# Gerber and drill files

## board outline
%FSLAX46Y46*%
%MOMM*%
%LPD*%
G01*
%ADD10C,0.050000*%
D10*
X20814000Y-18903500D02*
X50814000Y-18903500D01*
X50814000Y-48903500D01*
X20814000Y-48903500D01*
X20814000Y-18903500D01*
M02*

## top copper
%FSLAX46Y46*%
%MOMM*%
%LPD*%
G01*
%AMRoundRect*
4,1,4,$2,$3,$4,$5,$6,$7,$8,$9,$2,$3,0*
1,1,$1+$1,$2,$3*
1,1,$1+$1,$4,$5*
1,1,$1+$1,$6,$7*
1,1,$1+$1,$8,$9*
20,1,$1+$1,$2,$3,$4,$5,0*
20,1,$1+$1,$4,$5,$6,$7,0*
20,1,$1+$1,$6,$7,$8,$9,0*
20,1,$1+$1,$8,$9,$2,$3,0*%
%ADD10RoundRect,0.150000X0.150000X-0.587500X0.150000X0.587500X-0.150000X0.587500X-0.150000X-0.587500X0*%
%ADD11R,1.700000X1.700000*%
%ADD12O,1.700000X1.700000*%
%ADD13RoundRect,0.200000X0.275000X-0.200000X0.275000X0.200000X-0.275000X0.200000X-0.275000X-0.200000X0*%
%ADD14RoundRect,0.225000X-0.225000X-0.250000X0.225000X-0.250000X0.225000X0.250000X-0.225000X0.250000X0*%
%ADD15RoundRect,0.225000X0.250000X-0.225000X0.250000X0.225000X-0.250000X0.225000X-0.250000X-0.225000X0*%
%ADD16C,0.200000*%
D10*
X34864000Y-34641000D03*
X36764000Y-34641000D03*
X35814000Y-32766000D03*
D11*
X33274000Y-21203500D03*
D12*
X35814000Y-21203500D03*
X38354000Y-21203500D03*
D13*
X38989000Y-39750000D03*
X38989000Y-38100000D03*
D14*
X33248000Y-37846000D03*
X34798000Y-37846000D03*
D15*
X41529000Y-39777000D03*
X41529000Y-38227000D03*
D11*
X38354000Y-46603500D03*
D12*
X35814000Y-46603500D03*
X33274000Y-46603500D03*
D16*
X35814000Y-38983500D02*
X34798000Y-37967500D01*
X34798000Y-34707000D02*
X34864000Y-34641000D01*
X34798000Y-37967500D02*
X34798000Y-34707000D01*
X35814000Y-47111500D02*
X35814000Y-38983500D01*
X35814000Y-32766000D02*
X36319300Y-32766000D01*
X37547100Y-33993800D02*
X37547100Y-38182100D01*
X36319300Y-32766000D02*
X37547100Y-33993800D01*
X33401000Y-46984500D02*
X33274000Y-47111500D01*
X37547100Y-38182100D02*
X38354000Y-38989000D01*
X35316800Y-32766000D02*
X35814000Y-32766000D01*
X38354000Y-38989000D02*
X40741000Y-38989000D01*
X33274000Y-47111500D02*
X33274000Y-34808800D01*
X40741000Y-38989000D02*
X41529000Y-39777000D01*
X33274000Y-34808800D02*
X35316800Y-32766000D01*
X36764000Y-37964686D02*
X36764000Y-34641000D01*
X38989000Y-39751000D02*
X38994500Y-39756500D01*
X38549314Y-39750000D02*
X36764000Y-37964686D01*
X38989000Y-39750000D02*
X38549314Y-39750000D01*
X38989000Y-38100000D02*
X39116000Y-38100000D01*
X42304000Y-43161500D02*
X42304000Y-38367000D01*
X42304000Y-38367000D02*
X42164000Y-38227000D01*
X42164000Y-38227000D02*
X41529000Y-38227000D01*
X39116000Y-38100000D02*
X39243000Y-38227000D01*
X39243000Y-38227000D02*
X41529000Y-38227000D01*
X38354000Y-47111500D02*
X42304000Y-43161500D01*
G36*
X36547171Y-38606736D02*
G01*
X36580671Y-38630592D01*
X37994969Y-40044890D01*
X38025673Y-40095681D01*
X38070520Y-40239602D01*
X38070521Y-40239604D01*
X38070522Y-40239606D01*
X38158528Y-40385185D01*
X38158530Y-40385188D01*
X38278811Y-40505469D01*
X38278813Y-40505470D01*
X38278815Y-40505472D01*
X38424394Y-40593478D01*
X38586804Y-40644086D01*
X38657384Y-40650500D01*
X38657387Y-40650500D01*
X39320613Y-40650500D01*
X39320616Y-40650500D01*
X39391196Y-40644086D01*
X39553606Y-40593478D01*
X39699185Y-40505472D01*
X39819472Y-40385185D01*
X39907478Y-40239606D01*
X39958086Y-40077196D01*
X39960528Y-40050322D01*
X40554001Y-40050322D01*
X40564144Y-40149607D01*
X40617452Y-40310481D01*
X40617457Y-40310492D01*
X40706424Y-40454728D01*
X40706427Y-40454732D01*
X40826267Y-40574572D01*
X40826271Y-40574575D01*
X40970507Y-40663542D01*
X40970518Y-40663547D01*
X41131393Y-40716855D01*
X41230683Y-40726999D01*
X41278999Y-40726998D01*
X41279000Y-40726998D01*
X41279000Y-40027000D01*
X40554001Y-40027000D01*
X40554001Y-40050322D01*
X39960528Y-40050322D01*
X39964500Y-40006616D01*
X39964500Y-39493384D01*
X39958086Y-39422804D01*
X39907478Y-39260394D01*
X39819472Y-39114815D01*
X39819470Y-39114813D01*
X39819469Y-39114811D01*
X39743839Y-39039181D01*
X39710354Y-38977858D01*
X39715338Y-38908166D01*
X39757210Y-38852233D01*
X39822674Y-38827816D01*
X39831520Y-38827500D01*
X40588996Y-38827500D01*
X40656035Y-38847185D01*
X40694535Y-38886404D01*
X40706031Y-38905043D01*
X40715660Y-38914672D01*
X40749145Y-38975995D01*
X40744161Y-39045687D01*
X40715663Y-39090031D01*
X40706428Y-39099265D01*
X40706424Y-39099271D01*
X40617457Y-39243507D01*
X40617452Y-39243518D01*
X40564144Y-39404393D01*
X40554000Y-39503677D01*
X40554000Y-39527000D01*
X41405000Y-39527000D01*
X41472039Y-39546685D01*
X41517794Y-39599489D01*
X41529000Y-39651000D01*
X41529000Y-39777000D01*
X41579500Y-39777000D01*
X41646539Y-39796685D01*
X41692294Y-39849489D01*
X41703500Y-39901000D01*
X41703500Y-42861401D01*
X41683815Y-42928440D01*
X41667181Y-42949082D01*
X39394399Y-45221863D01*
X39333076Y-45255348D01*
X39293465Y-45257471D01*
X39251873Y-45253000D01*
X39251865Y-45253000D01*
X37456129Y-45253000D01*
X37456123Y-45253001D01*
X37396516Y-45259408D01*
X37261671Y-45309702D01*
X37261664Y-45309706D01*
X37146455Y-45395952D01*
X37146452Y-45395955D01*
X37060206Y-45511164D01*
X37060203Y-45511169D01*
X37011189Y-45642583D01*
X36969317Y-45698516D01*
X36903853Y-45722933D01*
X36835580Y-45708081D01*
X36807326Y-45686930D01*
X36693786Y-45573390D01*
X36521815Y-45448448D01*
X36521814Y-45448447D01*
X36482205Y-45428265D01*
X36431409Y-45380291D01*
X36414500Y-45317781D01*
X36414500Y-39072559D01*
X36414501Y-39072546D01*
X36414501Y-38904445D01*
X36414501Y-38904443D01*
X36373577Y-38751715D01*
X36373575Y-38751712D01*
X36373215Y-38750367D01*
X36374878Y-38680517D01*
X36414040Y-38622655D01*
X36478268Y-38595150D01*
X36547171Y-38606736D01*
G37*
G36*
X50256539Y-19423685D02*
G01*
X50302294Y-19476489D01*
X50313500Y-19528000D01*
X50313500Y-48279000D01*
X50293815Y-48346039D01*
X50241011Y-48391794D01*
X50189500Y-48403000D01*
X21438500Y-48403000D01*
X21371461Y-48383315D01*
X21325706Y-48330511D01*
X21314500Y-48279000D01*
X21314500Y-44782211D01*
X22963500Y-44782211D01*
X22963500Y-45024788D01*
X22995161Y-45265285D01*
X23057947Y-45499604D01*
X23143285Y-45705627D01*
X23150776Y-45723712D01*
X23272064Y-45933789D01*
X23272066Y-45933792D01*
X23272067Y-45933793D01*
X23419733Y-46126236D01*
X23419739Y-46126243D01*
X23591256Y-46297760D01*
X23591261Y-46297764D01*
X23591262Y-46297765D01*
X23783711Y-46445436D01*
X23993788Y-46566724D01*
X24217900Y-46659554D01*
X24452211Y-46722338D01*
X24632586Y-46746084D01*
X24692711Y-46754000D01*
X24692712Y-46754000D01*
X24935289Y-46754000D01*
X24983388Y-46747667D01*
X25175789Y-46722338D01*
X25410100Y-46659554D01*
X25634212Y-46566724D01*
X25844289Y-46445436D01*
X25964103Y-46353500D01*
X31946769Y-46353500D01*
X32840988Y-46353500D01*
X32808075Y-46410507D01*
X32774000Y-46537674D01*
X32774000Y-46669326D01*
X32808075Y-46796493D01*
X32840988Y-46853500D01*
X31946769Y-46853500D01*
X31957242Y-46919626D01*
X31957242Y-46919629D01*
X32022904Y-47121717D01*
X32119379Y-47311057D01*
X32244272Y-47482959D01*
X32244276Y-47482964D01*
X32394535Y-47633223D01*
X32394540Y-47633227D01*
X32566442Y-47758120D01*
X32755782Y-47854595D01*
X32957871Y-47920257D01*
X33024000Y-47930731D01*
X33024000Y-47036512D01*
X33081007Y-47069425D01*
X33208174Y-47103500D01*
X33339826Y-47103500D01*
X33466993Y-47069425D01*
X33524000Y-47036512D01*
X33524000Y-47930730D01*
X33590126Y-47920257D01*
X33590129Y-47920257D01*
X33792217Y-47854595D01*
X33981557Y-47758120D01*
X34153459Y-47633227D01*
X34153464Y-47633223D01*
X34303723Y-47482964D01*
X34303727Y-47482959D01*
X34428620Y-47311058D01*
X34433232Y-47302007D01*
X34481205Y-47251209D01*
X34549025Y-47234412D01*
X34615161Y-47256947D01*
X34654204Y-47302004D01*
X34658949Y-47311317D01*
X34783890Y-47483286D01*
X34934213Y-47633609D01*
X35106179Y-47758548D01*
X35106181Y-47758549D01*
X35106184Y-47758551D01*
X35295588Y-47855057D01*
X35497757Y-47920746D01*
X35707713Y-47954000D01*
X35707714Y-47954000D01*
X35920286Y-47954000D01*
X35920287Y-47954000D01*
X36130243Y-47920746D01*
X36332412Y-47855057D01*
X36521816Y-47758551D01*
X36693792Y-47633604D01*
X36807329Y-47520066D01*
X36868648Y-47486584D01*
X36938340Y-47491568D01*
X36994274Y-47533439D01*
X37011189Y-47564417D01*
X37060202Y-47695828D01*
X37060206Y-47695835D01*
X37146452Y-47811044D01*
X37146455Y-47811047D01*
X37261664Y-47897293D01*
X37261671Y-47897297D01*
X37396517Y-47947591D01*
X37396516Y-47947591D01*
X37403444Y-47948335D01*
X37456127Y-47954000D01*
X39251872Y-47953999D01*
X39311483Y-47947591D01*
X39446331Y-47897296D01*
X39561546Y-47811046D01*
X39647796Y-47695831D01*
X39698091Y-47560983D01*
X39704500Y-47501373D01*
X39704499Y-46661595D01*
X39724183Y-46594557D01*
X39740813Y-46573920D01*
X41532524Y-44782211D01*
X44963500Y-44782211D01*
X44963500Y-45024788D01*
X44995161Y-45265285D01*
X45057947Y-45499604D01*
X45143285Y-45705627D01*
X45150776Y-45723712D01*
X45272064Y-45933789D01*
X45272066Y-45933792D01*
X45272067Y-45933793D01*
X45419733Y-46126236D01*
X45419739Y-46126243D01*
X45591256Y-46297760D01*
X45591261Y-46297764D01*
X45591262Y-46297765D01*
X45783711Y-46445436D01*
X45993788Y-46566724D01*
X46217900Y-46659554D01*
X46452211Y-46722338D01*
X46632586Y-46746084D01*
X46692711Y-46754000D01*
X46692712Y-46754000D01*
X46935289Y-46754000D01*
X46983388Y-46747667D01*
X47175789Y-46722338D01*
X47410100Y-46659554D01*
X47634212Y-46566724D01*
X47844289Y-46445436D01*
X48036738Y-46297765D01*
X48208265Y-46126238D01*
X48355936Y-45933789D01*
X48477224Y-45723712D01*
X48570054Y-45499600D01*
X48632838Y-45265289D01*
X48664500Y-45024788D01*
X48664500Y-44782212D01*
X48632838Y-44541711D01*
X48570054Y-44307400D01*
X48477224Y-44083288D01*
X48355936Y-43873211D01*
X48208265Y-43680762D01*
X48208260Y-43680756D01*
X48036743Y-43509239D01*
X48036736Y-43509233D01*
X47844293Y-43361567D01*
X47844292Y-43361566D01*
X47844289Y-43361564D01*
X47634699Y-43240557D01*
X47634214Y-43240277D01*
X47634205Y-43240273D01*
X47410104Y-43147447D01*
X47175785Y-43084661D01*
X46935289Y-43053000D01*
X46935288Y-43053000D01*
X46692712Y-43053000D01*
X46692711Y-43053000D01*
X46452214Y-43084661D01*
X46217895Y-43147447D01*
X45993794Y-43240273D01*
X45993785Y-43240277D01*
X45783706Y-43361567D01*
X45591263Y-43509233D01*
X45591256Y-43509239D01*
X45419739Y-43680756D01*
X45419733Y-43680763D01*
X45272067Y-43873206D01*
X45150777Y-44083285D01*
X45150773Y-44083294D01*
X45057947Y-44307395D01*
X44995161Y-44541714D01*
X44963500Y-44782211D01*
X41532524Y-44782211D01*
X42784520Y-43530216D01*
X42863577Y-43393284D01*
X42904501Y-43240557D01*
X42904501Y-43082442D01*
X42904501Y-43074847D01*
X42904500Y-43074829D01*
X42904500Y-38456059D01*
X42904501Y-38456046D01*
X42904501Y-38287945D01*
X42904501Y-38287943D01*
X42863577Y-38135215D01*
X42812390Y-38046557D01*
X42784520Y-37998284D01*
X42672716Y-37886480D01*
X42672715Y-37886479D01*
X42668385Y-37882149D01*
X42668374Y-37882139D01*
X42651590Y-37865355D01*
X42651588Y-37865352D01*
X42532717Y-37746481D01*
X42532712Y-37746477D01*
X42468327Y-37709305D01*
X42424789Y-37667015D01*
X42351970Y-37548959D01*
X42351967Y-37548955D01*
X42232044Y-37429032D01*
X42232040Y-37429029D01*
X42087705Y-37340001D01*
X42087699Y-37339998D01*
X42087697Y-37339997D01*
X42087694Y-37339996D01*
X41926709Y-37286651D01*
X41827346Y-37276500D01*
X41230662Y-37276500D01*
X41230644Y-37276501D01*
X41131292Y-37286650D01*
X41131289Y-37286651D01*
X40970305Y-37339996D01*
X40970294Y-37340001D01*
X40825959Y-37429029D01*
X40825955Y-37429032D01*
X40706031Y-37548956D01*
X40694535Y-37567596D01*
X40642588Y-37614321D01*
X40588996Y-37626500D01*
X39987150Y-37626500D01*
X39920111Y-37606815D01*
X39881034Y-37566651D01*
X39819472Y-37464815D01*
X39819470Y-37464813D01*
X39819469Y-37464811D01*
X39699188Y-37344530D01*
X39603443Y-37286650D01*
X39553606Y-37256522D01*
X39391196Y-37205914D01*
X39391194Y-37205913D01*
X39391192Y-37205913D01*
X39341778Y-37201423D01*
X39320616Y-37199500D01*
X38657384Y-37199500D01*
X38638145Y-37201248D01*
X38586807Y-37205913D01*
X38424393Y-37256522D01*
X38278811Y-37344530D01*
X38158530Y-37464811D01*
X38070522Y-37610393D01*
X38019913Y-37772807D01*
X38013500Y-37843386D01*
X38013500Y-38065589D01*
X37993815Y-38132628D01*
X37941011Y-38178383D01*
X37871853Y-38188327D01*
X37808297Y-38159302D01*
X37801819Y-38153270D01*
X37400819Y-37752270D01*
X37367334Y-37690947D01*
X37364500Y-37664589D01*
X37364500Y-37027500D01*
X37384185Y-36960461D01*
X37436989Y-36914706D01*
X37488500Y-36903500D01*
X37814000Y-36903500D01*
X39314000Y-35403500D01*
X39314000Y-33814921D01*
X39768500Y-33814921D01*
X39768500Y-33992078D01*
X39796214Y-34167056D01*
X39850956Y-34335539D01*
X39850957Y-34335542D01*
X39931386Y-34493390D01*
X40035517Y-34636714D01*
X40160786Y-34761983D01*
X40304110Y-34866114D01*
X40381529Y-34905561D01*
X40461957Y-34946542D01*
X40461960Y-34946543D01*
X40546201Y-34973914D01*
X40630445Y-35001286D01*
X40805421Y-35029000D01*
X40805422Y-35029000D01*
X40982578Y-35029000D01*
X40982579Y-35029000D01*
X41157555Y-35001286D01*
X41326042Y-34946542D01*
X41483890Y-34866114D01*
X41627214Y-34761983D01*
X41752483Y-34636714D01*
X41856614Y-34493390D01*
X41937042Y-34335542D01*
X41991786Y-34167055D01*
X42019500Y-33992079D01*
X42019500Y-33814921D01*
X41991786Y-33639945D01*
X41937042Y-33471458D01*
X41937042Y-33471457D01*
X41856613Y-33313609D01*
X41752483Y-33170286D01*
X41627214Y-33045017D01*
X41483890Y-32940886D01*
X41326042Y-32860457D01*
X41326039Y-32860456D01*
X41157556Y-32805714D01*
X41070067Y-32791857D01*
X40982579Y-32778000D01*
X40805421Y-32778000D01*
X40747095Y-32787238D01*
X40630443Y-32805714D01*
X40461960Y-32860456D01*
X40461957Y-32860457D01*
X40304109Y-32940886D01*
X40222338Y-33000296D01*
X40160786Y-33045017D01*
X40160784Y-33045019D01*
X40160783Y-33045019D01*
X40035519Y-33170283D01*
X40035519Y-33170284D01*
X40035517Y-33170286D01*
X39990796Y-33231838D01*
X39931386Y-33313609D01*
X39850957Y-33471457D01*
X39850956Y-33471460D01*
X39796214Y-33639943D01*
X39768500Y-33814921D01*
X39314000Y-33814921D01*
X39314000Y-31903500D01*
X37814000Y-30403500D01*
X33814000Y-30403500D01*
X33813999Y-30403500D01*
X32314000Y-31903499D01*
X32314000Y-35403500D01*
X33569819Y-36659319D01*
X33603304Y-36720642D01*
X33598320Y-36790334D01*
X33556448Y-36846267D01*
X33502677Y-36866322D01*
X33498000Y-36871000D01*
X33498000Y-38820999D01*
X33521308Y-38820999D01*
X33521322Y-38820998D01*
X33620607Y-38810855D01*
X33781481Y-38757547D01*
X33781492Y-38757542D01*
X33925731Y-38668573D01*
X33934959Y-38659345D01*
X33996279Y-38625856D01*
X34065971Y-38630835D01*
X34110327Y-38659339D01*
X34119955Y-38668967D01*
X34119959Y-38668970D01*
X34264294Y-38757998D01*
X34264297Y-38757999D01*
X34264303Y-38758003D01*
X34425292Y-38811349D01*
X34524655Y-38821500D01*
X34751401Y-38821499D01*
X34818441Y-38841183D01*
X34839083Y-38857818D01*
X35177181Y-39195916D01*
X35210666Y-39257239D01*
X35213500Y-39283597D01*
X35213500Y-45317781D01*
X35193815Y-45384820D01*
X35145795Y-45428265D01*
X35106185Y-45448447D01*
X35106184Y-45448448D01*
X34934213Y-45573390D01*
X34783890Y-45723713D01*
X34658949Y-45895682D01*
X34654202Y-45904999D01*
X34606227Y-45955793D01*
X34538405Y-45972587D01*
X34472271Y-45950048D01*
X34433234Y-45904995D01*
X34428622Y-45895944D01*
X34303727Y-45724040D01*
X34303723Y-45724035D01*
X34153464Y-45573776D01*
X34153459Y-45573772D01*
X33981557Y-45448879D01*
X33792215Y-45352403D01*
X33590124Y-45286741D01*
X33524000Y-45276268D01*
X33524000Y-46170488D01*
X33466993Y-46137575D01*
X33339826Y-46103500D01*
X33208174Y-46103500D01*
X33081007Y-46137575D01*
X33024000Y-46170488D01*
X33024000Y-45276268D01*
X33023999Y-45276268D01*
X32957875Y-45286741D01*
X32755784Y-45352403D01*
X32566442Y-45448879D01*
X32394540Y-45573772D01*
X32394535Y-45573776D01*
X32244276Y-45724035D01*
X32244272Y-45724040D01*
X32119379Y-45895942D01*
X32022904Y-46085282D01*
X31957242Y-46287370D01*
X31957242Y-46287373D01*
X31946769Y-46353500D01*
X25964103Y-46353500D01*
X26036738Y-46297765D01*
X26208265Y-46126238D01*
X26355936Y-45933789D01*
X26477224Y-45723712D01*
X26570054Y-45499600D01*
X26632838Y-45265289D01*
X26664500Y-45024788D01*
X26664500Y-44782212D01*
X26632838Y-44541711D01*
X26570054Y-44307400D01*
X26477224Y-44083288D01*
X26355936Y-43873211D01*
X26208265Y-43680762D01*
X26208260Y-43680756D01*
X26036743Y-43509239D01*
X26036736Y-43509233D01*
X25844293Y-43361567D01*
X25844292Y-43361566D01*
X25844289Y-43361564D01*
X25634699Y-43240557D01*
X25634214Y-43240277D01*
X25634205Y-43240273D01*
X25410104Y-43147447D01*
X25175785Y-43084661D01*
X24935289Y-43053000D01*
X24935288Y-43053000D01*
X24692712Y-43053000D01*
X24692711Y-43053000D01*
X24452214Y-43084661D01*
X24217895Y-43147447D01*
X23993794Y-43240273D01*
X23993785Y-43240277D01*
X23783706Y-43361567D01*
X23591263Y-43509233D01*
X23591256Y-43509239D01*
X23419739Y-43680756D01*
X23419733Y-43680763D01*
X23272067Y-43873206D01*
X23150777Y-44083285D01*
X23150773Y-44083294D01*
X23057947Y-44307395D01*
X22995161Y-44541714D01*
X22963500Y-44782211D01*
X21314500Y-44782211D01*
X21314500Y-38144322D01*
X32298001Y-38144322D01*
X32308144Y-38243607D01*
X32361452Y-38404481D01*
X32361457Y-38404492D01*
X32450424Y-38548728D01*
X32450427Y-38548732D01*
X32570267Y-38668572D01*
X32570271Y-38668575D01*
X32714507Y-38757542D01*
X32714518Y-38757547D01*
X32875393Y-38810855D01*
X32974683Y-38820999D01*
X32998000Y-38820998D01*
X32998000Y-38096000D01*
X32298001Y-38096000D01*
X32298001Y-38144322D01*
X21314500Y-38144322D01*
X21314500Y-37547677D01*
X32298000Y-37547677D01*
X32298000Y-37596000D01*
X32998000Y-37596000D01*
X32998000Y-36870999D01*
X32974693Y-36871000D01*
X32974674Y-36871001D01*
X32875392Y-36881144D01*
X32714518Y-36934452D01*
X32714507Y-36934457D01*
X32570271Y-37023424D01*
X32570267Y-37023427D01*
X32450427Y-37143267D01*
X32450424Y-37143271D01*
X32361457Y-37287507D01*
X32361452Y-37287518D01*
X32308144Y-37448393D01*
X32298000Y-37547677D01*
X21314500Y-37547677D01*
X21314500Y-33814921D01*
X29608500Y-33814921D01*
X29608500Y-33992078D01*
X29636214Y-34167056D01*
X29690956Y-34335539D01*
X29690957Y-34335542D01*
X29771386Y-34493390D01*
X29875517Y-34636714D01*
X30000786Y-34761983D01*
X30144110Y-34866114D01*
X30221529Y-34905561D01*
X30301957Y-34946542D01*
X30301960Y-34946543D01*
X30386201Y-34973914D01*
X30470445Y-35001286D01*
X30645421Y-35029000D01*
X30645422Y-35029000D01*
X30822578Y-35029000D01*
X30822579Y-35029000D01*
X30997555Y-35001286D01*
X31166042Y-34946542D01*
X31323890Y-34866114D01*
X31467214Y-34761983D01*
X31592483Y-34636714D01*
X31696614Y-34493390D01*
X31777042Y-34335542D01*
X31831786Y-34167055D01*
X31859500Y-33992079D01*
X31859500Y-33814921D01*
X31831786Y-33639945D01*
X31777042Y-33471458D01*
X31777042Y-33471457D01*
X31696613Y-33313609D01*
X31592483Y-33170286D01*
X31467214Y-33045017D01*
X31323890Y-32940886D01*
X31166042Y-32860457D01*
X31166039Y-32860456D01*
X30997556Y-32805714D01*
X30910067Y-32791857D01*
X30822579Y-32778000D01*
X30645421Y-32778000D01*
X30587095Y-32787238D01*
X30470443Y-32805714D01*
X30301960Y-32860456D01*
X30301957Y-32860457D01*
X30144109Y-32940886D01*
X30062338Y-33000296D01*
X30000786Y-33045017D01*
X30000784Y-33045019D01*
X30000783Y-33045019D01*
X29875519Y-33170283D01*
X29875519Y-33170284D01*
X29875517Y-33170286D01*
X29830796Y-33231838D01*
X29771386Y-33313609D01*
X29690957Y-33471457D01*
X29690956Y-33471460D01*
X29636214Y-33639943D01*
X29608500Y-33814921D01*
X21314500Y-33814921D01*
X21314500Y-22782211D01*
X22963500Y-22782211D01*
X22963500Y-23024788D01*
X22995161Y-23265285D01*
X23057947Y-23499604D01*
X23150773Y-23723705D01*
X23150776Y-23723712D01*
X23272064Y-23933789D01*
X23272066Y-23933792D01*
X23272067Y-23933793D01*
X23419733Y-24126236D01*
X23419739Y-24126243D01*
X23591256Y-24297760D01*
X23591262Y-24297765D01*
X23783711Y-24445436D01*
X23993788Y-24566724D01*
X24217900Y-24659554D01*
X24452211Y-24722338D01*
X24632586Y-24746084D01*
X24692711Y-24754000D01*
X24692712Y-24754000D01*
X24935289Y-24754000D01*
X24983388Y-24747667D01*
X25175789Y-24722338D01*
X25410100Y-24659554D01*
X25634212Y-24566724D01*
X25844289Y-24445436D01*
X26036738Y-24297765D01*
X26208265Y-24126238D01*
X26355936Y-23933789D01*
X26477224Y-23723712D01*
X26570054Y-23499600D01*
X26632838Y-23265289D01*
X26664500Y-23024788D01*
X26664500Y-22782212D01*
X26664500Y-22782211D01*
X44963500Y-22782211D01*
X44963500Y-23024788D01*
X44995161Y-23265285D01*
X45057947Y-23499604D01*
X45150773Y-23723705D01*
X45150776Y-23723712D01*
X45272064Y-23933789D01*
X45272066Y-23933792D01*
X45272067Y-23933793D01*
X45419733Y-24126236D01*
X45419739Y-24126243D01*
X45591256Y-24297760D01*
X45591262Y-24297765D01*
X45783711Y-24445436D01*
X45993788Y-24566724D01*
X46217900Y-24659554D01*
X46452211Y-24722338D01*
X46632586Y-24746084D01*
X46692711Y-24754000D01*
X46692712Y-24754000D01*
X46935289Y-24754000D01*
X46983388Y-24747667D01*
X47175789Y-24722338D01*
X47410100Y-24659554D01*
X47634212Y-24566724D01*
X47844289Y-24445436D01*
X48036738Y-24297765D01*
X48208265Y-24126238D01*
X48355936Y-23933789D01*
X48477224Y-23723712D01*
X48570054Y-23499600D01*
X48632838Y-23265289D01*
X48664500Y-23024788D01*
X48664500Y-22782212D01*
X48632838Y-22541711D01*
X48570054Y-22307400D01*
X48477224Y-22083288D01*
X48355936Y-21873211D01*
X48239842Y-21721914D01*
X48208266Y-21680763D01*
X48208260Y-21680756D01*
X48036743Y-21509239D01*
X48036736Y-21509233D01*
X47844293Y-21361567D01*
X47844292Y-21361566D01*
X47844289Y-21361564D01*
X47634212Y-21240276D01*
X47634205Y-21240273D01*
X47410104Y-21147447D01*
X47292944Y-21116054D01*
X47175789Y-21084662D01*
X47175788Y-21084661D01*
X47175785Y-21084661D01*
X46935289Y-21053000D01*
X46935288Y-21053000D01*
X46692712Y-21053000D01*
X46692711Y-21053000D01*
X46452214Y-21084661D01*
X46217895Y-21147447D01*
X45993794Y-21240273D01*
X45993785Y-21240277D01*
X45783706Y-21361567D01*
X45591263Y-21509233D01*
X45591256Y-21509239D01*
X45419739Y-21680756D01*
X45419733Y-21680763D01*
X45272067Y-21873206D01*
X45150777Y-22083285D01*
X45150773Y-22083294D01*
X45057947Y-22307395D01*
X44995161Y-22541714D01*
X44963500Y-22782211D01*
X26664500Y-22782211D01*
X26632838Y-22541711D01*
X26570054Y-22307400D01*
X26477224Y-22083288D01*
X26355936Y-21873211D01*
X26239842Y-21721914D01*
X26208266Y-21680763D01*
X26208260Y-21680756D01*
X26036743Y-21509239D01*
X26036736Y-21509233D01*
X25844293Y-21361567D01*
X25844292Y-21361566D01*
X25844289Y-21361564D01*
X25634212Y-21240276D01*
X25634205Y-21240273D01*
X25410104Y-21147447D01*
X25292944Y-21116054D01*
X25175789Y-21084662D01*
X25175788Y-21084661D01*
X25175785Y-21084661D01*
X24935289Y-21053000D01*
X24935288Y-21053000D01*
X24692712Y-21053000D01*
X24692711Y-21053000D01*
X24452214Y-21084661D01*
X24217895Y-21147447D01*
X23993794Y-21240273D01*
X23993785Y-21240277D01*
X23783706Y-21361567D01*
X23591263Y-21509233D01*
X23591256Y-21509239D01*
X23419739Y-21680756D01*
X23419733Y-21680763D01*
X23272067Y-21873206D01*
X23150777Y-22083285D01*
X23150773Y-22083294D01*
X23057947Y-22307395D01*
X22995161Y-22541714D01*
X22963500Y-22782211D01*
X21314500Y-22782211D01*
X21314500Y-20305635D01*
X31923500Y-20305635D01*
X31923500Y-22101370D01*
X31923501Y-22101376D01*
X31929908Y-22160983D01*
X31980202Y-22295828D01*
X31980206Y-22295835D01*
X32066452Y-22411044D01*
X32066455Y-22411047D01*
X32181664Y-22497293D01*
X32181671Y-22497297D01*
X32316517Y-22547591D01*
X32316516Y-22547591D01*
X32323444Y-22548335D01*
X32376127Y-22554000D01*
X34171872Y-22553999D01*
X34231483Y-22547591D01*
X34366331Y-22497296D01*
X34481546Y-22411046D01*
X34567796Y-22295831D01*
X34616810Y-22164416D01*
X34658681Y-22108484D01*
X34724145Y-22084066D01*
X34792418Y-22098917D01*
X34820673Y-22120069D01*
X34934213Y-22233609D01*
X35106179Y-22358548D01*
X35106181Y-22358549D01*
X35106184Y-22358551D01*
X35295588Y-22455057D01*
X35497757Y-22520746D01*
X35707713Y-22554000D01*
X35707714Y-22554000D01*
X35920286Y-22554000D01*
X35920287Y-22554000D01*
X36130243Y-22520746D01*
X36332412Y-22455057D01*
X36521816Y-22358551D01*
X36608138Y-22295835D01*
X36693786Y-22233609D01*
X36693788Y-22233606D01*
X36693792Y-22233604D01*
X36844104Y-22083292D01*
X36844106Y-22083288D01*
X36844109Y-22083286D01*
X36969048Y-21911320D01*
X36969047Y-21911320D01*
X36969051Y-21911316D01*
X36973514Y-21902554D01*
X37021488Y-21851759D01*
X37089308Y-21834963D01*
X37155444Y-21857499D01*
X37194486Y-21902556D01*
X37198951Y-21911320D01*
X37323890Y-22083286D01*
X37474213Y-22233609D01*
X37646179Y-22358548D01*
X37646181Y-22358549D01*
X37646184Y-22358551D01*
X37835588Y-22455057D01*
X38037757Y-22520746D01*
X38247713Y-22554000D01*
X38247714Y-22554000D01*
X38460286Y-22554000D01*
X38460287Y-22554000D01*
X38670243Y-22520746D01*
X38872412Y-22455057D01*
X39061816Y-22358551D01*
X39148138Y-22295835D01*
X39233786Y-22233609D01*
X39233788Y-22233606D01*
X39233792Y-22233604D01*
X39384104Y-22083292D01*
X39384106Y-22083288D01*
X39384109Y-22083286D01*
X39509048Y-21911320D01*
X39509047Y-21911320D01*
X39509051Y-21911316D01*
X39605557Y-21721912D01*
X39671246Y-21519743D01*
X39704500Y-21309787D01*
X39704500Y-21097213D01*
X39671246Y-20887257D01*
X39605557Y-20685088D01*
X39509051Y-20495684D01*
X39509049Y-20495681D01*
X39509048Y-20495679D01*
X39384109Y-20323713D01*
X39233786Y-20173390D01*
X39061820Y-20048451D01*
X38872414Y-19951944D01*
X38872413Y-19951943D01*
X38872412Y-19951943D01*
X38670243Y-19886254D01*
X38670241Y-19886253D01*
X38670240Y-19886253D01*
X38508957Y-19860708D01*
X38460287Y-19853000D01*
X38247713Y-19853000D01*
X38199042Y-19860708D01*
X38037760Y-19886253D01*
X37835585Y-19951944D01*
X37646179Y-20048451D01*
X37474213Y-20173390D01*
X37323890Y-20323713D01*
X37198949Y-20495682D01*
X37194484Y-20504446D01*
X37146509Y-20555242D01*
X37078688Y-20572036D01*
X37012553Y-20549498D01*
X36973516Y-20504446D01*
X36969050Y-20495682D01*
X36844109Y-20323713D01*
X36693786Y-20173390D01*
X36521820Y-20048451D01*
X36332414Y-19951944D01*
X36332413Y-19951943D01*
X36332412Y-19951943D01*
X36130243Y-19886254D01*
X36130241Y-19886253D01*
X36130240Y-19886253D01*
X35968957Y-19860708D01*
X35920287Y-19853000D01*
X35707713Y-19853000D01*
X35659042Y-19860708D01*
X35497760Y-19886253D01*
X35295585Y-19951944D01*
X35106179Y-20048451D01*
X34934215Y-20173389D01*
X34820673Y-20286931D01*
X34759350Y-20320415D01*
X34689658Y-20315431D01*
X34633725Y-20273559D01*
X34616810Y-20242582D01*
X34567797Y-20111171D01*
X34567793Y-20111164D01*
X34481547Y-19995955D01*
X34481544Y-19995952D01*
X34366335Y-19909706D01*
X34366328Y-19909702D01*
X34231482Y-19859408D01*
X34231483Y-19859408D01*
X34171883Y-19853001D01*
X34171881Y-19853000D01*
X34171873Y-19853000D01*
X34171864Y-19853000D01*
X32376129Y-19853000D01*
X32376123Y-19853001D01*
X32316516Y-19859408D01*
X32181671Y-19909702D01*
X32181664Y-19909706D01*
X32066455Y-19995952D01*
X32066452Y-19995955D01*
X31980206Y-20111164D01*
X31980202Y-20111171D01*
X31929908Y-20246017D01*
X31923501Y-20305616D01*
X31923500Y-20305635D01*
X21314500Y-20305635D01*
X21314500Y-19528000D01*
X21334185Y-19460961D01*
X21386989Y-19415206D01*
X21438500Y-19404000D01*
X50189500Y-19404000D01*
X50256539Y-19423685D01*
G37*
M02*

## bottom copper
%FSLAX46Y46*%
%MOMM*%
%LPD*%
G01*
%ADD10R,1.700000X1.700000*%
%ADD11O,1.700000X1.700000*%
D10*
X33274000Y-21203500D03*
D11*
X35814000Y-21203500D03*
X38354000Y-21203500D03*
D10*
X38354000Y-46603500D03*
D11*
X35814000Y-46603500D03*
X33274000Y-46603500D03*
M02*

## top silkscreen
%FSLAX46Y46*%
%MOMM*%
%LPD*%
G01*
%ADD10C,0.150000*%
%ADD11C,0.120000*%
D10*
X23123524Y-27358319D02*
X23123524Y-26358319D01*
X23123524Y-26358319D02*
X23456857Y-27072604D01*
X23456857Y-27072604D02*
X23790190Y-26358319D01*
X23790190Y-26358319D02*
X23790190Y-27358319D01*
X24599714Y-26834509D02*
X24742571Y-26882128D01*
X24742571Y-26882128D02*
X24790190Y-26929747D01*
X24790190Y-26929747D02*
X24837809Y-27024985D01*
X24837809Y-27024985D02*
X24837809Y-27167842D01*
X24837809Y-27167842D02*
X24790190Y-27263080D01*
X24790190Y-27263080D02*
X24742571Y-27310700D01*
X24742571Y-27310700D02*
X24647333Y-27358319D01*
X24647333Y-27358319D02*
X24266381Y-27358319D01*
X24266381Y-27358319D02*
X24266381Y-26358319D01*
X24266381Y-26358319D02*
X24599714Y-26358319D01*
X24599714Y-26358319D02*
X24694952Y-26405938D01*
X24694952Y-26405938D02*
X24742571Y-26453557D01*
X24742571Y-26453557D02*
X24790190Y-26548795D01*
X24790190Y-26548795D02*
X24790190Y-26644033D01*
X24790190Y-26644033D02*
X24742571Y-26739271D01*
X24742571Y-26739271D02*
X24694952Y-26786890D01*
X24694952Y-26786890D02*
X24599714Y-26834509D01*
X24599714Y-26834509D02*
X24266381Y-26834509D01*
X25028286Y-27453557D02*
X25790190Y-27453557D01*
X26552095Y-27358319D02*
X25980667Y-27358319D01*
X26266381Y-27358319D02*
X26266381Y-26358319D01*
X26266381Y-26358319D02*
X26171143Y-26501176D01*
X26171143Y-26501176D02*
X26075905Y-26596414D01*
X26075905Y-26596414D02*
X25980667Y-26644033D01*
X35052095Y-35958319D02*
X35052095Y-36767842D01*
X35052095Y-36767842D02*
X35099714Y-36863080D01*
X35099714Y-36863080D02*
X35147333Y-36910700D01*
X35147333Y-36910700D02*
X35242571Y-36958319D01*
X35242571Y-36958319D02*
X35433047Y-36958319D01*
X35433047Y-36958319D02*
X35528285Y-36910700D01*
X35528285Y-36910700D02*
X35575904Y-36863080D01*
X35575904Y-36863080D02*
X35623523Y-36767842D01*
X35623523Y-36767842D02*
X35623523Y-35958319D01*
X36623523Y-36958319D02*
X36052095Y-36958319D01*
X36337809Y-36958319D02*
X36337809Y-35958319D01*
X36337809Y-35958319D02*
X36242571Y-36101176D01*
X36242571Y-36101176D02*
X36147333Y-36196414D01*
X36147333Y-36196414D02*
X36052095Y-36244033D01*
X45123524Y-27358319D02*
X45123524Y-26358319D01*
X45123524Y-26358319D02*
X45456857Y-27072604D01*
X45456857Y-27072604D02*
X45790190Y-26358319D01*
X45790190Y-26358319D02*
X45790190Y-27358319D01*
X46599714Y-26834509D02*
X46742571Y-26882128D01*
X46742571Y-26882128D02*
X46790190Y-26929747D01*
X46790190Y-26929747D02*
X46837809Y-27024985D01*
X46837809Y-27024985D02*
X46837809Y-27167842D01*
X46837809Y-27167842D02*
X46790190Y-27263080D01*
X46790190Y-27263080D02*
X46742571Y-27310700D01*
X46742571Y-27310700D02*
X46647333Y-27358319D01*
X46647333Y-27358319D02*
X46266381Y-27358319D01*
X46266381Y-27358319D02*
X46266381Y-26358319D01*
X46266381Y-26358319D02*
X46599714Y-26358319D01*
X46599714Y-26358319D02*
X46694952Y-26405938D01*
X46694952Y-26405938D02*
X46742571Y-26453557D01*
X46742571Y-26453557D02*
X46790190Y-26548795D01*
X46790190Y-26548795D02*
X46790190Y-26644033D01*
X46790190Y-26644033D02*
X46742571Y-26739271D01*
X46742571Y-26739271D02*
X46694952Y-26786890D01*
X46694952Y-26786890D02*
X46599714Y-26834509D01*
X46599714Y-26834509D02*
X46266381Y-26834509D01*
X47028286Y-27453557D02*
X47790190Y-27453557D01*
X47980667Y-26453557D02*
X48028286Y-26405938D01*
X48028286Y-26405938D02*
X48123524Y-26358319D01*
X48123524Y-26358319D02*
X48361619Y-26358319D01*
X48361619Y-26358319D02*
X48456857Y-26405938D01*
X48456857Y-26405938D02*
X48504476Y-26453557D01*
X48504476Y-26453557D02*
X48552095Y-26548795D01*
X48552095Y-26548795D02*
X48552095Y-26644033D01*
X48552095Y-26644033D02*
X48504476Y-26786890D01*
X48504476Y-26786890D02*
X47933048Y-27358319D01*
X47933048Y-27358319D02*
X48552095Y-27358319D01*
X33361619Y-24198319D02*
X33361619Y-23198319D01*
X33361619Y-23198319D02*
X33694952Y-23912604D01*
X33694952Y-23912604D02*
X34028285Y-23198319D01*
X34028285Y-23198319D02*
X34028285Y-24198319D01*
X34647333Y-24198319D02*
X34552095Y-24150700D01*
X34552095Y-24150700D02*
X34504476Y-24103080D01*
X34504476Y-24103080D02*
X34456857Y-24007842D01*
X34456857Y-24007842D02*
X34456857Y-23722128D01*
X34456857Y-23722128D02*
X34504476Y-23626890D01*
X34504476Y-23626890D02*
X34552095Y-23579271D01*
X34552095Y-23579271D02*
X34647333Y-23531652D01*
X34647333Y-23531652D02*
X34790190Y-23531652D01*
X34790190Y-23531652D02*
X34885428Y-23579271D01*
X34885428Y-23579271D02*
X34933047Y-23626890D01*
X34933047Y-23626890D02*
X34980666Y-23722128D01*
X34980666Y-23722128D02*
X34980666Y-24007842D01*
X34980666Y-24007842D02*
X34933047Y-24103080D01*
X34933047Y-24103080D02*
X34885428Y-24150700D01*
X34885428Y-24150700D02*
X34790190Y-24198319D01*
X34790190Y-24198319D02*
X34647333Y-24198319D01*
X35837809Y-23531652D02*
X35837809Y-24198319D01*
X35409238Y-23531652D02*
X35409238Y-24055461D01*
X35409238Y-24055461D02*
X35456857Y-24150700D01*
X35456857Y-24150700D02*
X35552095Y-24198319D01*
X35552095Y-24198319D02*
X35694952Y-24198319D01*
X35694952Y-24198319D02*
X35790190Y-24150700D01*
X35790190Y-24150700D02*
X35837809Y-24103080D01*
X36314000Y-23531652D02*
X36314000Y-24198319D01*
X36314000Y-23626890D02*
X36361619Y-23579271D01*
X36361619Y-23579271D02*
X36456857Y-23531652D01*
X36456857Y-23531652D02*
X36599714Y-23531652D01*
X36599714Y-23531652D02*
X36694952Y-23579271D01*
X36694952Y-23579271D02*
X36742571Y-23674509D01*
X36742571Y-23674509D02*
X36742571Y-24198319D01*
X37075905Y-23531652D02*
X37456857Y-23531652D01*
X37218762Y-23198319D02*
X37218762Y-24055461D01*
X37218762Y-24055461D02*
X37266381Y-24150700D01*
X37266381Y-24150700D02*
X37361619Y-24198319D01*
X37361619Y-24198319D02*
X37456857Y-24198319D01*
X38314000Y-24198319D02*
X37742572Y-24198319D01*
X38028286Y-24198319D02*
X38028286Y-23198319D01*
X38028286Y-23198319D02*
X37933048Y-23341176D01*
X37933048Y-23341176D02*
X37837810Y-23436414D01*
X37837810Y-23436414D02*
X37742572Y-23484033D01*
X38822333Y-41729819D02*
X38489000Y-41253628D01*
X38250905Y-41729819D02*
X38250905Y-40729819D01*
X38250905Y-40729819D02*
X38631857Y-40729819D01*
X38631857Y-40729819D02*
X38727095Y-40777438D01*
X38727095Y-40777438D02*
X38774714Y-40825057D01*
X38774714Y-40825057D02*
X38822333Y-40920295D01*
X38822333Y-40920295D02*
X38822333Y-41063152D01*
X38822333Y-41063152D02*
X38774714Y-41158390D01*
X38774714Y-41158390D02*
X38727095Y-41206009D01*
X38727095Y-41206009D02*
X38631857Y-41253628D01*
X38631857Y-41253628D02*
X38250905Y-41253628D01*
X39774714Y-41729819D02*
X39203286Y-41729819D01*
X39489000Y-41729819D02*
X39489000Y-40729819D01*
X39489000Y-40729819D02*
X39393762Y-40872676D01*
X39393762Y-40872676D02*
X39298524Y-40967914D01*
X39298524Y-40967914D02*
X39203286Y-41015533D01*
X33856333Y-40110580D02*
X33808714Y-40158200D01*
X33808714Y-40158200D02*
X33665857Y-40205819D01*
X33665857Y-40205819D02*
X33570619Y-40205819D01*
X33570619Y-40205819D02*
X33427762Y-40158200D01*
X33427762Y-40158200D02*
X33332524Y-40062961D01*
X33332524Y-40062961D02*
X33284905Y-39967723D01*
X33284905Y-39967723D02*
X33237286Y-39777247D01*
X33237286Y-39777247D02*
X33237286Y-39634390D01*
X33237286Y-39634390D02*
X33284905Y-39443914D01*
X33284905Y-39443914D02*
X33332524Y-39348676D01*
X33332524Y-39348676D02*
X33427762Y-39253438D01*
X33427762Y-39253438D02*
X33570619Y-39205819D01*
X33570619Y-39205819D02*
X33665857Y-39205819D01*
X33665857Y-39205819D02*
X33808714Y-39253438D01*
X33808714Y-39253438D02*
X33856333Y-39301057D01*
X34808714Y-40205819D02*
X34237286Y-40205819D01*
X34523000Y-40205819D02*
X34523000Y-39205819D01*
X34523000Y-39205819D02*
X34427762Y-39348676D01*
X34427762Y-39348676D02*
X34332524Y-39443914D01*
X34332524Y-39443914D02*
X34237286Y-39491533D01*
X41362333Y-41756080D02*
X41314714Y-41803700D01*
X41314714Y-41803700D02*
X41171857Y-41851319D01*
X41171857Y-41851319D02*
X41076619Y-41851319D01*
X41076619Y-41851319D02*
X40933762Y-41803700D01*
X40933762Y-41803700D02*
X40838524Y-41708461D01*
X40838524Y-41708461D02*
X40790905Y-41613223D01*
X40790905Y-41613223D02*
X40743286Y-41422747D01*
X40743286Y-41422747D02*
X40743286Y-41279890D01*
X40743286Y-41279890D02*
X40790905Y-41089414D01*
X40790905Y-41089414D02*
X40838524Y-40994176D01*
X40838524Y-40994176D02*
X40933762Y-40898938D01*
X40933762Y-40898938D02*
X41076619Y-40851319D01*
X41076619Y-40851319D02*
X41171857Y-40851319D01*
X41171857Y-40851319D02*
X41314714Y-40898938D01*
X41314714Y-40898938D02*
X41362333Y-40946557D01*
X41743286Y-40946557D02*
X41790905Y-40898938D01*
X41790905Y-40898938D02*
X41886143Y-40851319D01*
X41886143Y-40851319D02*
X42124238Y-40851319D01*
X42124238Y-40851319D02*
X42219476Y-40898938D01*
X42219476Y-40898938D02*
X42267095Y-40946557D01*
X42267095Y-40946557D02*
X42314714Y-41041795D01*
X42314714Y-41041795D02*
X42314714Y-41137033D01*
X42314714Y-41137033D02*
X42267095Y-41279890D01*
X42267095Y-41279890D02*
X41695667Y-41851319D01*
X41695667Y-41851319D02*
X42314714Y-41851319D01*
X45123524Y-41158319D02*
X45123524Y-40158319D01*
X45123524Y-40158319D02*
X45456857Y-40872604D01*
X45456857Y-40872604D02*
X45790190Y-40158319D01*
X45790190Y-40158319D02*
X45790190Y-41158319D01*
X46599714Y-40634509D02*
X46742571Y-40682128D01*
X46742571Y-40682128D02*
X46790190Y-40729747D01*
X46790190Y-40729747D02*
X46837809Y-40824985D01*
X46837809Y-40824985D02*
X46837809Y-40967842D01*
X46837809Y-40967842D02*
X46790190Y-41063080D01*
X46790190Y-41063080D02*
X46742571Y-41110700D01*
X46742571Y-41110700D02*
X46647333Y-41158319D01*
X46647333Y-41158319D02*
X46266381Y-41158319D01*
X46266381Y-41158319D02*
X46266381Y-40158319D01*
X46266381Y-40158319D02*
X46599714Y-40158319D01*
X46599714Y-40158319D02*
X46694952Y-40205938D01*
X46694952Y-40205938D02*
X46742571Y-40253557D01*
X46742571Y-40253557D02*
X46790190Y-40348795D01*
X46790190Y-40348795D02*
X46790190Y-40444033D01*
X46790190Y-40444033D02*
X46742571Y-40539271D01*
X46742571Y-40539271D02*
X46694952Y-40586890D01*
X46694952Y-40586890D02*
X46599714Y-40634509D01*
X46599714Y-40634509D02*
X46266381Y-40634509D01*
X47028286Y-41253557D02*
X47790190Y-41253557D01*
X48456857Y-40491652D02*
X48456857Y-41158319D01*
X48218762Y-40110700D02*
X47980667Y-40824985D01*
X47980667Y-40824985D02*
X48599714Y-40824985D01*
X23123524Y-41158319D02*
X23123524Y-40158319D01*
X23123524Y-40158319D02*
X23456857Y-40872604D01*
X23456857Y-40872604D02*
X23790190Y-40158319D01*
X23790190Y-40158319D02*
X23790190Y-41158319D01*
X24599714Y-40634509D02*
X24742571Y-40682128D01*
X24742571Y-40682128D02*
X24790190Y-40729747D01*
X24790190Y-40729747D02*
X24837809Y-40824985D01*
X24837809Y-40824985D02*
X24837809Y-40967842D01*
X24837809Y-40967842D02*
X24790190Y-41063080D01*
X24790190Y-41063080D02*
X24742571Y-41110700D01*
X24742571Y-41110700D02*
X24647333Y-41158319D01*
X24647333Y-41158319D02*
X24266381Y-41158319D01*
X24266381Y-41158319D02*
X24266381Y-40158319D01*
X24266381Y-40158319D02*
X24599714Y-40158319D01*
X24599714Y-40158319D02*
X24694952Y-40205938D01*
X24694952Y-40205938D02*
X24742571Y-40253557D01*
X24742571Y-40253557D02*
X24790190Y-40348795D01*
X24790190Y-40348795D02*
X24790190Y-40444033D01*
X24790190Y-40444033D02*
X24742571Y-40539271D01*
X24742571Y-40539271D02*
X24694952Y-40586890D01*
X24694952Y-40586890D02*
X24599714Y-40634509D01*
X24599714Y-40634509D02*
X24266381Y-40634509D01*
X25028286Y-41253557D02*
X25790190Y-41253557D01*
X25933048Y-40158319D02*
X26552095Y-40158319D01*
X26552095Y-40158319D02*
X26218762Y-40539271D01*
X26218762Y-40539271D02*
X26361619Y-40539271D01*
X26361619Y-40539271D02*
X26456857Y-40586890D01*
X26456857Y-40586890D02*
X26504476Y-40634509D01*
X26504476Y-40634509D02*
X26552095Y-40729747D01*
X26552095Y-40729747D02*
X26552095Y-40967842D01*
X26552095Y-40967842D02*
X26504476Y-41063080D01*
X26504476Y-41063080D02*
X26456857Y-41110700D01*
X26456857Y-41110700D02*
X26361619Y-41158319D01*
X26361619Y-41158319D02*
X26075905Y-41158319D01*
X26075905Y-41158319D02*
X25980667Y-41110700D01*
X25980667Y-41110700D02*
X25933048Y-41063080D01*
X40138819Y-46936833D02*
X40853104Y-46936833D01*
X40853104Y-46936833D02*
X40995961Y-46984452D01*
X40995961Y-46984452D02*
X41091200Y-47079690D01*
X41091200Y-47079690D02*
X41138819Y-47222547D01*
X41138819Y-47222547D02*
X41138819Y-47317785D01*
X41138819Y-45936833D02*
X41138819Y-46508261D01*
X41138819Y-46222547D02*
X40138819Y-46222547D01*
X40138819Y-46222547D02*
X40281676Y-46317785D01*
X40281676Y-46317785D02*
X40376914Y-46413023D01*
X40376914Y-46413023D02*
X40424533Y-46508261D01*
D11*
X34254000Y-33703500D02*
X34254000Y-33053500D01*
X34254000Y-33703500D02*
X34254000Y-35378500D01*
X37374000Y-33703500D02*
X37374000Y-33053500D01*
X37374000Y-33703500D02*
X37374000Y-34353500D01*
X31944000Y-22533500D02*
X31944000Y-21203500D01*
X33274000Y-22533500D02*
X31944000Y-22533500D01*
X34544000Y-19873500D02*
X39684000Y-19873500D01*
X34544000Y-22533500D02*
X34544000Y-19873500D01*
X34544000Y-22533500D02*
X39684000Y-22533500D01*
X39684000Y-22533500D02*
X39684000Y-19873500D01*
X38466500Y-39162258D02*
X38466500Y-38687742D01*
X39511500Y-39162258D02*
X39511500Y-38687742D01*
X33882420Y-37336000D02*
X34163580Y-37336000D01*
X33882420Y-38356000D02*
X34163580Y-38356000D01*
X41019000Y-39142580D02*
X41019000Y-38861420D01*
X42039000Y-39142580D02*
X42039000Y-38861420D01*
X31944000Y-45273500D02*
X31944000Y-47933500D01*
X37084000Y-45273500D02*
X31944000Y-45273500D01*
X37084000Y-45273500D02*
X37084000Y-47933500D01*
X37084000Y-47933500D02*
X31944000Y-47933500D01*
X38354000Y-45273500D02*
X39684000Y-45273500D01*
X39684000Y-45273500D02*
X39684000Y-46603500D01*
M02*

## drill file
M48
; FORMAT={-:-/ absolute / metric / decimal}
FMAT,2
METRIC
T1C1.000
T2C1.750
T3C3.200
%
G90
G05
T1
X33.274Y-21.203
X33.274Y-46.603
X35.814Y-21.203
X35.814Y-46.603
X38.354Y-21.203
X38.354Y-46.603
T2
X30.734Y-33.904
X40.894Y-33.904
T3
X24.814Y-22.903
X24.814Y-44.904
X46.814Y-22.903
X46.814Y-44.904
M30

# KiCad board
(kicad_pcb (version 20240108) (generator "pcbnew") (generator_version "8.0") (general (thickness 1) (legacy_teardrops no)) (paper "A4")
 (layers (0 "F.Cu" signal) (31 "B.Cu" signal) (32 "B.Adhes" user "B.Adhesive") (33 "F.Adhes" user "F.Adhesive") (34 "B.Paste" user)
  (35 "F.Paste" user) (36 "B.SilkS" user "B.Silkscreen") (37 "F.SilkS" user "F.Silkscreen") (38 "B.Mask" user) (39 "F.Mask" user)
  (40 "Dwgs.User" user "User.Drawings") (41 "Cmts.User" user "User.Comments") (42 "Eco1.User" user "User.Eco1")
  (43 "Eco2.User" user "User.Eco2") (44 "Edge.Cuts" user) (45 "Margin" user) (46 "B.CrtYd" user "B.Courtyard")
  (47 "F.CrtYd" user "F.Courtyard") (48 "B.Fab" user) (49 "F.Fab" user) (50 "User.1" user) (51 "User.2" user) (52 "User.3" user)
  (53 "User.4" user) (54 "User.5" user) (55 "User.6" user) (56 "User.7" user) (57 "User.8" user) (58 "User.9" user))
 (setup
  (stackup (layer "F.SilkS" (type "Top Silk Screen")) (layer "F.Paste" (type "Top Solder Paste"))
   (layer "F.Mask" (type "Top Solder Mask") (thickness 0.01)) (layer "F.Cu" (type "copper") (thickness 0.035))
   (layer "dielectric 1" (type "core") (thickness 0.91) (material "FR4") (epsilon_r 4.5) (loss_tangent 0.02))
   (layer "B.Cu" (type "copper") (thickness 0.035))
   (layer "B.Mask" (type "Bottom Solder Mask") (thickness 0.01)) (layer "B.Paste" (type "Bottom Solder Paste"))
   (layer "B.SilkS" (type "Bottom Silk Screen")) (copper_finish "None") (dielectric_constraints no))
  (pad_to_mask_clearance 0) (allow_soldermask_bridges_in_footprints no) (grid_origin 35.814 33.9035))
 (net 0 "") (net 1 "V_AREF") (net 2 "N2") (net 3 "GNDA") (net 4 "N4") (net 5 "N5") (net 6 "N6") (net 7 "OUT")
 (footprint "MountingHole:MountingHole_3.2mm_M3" (layer "F.Cu") (at 24.814 22.9035)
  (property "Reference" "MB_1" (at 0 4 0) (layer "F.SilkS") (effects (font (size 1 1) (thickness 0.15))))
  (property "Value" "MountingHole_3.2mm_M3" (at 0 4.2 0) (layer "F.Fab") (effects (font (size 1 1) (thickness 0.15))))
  (pad "" np_thru_hole circle (at 0 0) (size 3.2 3.2) (drill 3.2) (layers "*.Cu" "*.Mask")))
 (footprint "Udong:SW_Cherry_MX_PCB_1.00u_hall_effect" (layer "F.Cu") (at 35.814 33.9035 180)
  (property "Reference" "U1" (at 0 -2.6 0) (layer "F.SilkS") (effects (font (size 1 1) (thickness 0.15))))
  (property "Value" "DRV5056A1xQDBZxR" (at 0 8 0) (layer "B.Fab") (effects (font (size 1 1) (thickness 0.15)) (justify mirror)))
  (fp_line (start 1.56 0.2) (end 1.56 0.85) (stroke (width 0.12) (type solid)) (layer "F.SilkS"))
  (fp_line (start 1.56 0.2) (end 1.56 -1.475) (stroke (width 0.12) (type solid)) (layer "F.SilkS"))
  (fp_line (start -1.56 0.2) (end -1.56 0.85) (stroke (width 0.12) (type solid)) (layer "F.SilkS"))
  (fp_line (start -1.56 0.2) (end -1.56 -0.45) (stroke (width 0.12) (type solid)) (layer "F.SilkS"))
  (pad "" np_thru_hole circle (at -5.08 0 180) (size 1.75 1.75) (drill 1.75) (layers "*.Cu" "*.Mask"))
  (pad "" np_thru_hole circle (at 5.08 0 180) (size 1.75 1.75) (drill 1.75) (layers "*.Cu" "*.Mask"))
  (pad "1" smd roundrect (at 0.95 -0.7375 90) (size 1.475 0.6) (layers "F.Cu" "F.Paste" "F.Mask") (roundrect_rratio 0.25) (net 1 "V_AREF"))
  (pad "2" smd roundrect (at -0.95 -0.7375 90) (size 1.475 0.6) (layers "F.Cu" "F.Paste" "F.Mask") (roundrect_rratio 0.25) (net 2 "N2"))
  (pad "3" smd roundrect (at 0 1.1375 90) (size 1.475 0.6) (layers "F.Cu" "F.Paste" "F.Mask") (roundrect_rratio 0.25) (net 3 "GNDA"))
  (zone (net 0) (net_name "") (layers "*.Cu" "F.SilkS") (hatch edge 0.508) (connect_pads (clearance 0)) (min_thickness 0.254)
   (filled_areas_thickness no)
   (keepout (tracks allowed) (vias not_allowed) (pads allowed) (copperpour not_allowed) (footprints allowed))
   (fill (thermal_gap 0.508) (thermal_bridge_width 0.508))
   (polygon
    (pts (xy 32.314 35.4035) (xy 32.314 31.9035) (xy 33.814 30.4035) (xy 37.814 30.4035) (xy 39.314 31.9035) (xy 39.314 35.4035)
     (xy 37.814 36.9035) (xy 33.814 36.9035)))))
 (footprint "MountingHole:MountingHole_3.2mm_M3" (layer "F.Cu") (at 46.814 22.9035)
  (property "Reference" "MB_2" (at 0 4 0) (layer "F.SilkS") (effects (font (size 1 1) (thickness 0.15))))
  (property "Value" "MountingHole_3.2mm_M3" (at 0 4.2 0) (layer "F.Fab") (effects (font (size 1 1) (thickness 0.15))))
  (pad "" np_thru_hole circle (at 0 0) (size 3.2 3.2) (drill 3.2) (layers "F&B.Cu" "*.Mask")))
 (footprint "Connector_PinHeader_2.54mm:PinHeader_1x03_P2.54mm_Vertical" (layer "F.Cu") (at 33.274 21.2035 90)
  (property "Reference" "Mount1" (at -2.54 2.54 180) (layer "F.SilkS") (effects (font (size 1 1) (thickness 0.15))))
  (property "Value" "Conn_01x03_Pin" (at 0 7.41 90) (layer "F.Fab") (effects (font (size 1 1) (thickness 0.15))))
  (fp_line (start -1.33 -1.33) (end 0 -1.33) (stroke (width 0.12) (type solid)) (layer "F.SilkS"))
  (fp_line (start -1.33 0) (end -1.33 -1.33) (stroke (width 0.12) (type solid)) (layer "F.SilkS"))
  (fp_line (start 1.33 1.27) (end 1.33 6.41) (stroke (width 0.12) (type solid)) (layer "F.SilkS"))
  (fp_line (start -1.33 1.27) (end 1.33 1.27) (stroke (width 0.12) (type solid)) (layer "F.SilkS"))
  (fp_line (start -1.33 1.27) (end -1.33 6.41) (stroke (width 0.12) (type solid)) (layer "F.SilkS"))
  (fp_line (start -1.33 6.41) (end 1.33 6.41) (stroke (width 0.12) (type solid)) (layer "F.SilkS"))
  (pad "1" thru_hole rect (at 0 0 90) (size 1.7 1.7) (drill 1) (layers "*.Cu" "*.Mask") (remove_unused_layers no) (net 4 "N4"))
  (pad "2" thru_hole oval (at 0 2.54 90) (size 1.7 1.7) (drill 1) (layers "*.Cu" "*.Mask") (remove_unused_layers no) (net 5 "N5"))
  (pad "3" thru_hole oval (at 0 5.08 90) (size 1.7 1.7) (drill 1) (layers "*.Cu" "*.Mask") (remove_unused_layers no) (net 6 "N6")))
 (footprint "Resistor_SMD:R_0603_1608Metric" (layer "F.Cu") (at 38.989 38.925 90)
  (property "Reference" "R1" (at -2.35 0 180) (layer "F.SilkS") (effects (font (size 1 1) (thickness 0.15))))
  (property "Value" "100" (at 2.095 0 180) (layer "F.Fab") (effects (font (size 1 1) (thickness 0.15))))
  (fp_line (start -0.237258 -0.5225) (end 0.237258 -0.5225) (stroke (width 0.12) (type solid)) (layer "F.SilkS"))
  (fp_line (start -0.237258 0.5225) (end 0.237258 0.5225) (stroke (width 0.12) (type solid)) (layer "F.SilkS"))
  (pad "1" smd roundrect (at -0.825 0 90) (size 0.8 0.95) (layers "F.Cu" "F.Paste" "F.Mask") (roundrect_rratio 0.25) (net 2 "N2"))
  (pad "2" smd roundrect (at 0.825 0 90) (size 0.8 0.95) (layers "F.Cu" "F.Paste" "F.Mask") (roundrect_rratio 0.25) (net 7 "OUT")))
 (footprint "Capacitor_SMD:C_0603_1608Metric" (layer "F.Cu") (at 34.023 37.846)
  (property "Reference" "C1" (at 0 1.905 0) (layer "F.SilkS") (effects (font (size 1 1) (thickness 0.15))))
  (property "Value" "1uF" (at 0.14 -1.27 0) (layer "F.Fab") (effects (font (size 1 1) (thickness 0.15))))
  (fp_line (start -0.14058 -0.51) (end 0.14058 -0.51) (stroke (width 0.12) (type solid)) (layer "F.SilkS"))
  (fp_line (start -0.14058 0.51) (end 0.14058 0.51) (stroke (width 0.12) (type solid)) (layer "F.SilkS"))
  (pad "1" smd roundrect (at -0.775 0) (size 0.9 0.95) (layers "F.Cu" "F.Paste" "F.Mask") (roundrect_rratio 0.25) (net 3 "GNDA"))
  (pad "2" smd roundrect (at 0.775 0) (size 0.9 0.95) (layers "F.Cu" "F.Paste" "F.Mask") (roundrect_rratio 0.25) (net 1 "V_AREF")))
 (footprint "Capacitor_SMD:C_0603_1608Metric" (layer "F.Cu") (at 41.529 39.002 90)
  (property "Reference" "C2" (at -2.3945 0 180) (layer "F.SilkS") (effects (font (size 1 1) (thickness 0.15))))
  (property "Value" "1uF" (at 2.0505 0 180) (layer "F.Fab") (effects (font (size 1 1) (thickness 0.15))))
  (fp_line (start -0.14058 -0.51) (end 0.14058 -0.51) (stroke (width 0.12) (type solid)) (layer "F.SilkS"))
  (fp_line (start -0.14058 0.51) (end 0.14058 0.51) (stroke (width 0.12) (type solid)) (layer "F.SilkS"))
  (pad "1" smd roundrect (at -0.775 0 90) (size 0.9 0.95) (layers "F.Cu" "F.Paste" "F.Mask") (roundrect_rratio 0.25) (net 3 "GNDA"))
  (pad "2" smd roundrect (at 0.775 0 90) (size 0.9 0.95) (layers "F.Cu" "F.Paste" "F.Mask") (roundrect_rratio 0.25) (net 7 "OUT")))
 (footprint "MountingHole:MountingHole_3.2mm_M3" (layer "F.Cu") (at 46.814 44.9035)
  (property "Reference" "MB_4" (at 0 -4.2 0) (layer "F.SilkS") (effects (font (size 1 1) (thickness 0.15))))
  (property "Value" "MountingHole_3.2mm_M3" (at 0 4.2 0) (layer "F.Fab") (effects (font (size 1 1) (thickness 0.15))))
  (pad "" np_thru_hole circle (at 0 0) (size 3.2 3.2) (drill 3.2) (layers "F&B.Cu" "*.Mask")))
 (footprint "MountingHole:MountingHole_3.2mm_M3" (layer "F.Cu") (at 24.814 44.9035)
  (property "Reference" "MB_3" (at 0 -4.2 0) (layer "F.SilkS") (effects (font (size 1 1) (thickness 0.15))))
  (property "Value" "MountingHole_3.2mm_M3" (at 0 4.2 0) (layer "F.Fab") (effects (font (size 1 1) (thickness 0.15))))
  (pad "" np_thru_hole circle (at 0 0) (size 3.2 3.2) (drill 3.2) (layers "F&B.Cu" "*.Mask")))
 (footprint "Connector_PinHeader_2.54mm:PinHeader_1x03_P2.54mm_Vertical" (layer "F.Cu") (at 38.354 46.6035 -90)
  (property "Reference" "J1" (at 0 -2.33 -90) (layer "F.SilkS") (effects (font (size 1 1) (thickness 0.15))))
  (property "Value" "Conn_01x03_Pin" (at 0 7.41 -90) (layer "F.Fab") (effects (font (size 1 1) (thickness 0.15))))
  (fp_line (start -1.33 6.41) (end 1.33 6.41) (stroke (width 0.12) (type solid)) (layer "F.SilkS"))
  (fp_line (start -1.33 1.27) (end -1.33 6.41) (stroke (width 0.12) (type solid)) (layer "F.SilkS"))
  (fp_line (start -1.33 1.27) (end 1.33 1.27) (stroke (width 0.12) (type solid)) (layer "F.SilkS"))
  (fp_line (start 1.33 1.27) (end 1.33 6.41) (stroke (width 0.12) (type solid)) (layer "F.SilkS"))
  (fp_line (start -1.33 0) (end -1.33 -1.33) (stroke (width 0.12) (type solid)) (layer "F.SilkS"))
  (fp_line (start -1.33 -1.33) (end 0 -1.33) (stroke (width 0.12) (type solid)) (layer "F.SilkS"))
  (pad "1" thru_hole rect (at 0 0 270) (size 1.7 1.7) (drill 1) (layers "*.Cu" "*.Mask") (remove_unused_layers no) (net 7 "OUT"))
  (pad "2" thru_hole oval (at 0 2.54 270) (size 1.7 1.7) (drill 1) (layers "*.Cu" "*.Mask") (remove_unused_layers no) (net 1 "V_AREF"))
  (pad "3" thru_hole oval (at 0 5.08 270) (size 1.7 1.7) (drill 1) (layers "*.Cu" "*.Mask") (remove_unused_layers no) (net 3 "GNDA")))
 (gr_rect (start 20.814 18.9035) (end 50.814 48.9035) (stroke (width 0.05) (type default)) (fill none) (layer "Edge.Cuts"))
 (segment (start 35.814 38.9835) (end 34.798 37.9675) (width 0.2) (layer "F.Cu") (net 1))
 (segment (start 34.798 34.707) (end 34.864 34.641) (width 0.2) (layer "F.Cu") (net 1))
 (segment (start 34.798 37.9675) (end 34.798 34.707) (width 0.2) (layer "F.Cu") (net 1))
 (segment (start 35.814 47.1115) (end 35.814 38.9835) (width 0.2) (layer "F.Cu") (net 1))
 (segment (start 35.814 32.766) (end 36.3193 32.766) (width 0.2) (layer "F.Cu") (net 3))
 (segment (start 37.5471 33.9938) (end 37.5471 38.1821) (width 0.2) (layer "F.Cu") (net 3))
 (segment (start 36.3193 32.766) (end 37.5471 33.9938) (width 0.2) (layer "F.Cu") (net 3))
 (segment (start 33.401 46.9845) (end 33.274 47.1115) (width 0.2) (layer "F.Cu") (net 3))
 (segment (start 37.5471 38.1821) (end 38.354 38.989) (width 0.2) (layer "F.Cu") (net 3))
 (segment (start 35.3168 32.766) (end 35.814 32.766) (width 0.2) (layer "F.Cu") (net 3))
 (segment (start 38.354 38.989) (end 40.741 38.989) (width 0.2) (layer "F.Cu") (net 3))
 (segment (start 33.274 47.1115) (end 33.274 34.8088) (width 0.2) (layer "F.Cu") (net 3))
 (segment (start 40.741 38.989) (end 41.529 39.777) (width 0.2) (layer "F.Cu") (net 3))
 (segment (start 33.274 34.8088) (end 35.3168 32.766) (width 0.2) (layer "F.Cu") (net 3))
 (segment (start 36.764 37.964686) (end 36.764 34.641) (width 0.2) (layer "F.Cu") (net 2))
 (segment (start 38.989 39.751) (end 38.9945 39.7565) (width 0.2) (layer "F.Cu") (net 2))
 (segment (start 38.549314 39.75) (end 36.764 37.964686) (width 0.2) (layer "F.Cu") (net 2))
 (segment (start 38.989 39.75) (end 38.549314 39.75) (width 0.2) (layer "F.Cu") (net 2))
 (segment (start 38.989 38.1) (end 39.116 38.1) (width 0.2) (layer "F.Cu") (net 7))
 (segment (start 42.304 43.1615) (end 42.304 38.367) (width 0.2) (layer "F.Cu") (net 7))
 (segment (start 42.304 38.367) (end 42.164 38.227) (width 0.2) (layer "F.Cu") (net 7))
 (segment (start 42.164 38.227) (end 41.529 38.227) (width 0.2) (layer "F.Cu") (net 7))
 (segment (start 39.116 38.1) (end 39.243 38.227) (width 0.2) (layer "F.Cu") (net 7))
 (segment (start 39.243 38.227) (end 41.529 38.227) (width 0.2) (layer "F.Cu") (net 7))
 (segment (start 38.354 47.1115) (end 42.304 43.1615) (width 0.2) (layer "F.Cu") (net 7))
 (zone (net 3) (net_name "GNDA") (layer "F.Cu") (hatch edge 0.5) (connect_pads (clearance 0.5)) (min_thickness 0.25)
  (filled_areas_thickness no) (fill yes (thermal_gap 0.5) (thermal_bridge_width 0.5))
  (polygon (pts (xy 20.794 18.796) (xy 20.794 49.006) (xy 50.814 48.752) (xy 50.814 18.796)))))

